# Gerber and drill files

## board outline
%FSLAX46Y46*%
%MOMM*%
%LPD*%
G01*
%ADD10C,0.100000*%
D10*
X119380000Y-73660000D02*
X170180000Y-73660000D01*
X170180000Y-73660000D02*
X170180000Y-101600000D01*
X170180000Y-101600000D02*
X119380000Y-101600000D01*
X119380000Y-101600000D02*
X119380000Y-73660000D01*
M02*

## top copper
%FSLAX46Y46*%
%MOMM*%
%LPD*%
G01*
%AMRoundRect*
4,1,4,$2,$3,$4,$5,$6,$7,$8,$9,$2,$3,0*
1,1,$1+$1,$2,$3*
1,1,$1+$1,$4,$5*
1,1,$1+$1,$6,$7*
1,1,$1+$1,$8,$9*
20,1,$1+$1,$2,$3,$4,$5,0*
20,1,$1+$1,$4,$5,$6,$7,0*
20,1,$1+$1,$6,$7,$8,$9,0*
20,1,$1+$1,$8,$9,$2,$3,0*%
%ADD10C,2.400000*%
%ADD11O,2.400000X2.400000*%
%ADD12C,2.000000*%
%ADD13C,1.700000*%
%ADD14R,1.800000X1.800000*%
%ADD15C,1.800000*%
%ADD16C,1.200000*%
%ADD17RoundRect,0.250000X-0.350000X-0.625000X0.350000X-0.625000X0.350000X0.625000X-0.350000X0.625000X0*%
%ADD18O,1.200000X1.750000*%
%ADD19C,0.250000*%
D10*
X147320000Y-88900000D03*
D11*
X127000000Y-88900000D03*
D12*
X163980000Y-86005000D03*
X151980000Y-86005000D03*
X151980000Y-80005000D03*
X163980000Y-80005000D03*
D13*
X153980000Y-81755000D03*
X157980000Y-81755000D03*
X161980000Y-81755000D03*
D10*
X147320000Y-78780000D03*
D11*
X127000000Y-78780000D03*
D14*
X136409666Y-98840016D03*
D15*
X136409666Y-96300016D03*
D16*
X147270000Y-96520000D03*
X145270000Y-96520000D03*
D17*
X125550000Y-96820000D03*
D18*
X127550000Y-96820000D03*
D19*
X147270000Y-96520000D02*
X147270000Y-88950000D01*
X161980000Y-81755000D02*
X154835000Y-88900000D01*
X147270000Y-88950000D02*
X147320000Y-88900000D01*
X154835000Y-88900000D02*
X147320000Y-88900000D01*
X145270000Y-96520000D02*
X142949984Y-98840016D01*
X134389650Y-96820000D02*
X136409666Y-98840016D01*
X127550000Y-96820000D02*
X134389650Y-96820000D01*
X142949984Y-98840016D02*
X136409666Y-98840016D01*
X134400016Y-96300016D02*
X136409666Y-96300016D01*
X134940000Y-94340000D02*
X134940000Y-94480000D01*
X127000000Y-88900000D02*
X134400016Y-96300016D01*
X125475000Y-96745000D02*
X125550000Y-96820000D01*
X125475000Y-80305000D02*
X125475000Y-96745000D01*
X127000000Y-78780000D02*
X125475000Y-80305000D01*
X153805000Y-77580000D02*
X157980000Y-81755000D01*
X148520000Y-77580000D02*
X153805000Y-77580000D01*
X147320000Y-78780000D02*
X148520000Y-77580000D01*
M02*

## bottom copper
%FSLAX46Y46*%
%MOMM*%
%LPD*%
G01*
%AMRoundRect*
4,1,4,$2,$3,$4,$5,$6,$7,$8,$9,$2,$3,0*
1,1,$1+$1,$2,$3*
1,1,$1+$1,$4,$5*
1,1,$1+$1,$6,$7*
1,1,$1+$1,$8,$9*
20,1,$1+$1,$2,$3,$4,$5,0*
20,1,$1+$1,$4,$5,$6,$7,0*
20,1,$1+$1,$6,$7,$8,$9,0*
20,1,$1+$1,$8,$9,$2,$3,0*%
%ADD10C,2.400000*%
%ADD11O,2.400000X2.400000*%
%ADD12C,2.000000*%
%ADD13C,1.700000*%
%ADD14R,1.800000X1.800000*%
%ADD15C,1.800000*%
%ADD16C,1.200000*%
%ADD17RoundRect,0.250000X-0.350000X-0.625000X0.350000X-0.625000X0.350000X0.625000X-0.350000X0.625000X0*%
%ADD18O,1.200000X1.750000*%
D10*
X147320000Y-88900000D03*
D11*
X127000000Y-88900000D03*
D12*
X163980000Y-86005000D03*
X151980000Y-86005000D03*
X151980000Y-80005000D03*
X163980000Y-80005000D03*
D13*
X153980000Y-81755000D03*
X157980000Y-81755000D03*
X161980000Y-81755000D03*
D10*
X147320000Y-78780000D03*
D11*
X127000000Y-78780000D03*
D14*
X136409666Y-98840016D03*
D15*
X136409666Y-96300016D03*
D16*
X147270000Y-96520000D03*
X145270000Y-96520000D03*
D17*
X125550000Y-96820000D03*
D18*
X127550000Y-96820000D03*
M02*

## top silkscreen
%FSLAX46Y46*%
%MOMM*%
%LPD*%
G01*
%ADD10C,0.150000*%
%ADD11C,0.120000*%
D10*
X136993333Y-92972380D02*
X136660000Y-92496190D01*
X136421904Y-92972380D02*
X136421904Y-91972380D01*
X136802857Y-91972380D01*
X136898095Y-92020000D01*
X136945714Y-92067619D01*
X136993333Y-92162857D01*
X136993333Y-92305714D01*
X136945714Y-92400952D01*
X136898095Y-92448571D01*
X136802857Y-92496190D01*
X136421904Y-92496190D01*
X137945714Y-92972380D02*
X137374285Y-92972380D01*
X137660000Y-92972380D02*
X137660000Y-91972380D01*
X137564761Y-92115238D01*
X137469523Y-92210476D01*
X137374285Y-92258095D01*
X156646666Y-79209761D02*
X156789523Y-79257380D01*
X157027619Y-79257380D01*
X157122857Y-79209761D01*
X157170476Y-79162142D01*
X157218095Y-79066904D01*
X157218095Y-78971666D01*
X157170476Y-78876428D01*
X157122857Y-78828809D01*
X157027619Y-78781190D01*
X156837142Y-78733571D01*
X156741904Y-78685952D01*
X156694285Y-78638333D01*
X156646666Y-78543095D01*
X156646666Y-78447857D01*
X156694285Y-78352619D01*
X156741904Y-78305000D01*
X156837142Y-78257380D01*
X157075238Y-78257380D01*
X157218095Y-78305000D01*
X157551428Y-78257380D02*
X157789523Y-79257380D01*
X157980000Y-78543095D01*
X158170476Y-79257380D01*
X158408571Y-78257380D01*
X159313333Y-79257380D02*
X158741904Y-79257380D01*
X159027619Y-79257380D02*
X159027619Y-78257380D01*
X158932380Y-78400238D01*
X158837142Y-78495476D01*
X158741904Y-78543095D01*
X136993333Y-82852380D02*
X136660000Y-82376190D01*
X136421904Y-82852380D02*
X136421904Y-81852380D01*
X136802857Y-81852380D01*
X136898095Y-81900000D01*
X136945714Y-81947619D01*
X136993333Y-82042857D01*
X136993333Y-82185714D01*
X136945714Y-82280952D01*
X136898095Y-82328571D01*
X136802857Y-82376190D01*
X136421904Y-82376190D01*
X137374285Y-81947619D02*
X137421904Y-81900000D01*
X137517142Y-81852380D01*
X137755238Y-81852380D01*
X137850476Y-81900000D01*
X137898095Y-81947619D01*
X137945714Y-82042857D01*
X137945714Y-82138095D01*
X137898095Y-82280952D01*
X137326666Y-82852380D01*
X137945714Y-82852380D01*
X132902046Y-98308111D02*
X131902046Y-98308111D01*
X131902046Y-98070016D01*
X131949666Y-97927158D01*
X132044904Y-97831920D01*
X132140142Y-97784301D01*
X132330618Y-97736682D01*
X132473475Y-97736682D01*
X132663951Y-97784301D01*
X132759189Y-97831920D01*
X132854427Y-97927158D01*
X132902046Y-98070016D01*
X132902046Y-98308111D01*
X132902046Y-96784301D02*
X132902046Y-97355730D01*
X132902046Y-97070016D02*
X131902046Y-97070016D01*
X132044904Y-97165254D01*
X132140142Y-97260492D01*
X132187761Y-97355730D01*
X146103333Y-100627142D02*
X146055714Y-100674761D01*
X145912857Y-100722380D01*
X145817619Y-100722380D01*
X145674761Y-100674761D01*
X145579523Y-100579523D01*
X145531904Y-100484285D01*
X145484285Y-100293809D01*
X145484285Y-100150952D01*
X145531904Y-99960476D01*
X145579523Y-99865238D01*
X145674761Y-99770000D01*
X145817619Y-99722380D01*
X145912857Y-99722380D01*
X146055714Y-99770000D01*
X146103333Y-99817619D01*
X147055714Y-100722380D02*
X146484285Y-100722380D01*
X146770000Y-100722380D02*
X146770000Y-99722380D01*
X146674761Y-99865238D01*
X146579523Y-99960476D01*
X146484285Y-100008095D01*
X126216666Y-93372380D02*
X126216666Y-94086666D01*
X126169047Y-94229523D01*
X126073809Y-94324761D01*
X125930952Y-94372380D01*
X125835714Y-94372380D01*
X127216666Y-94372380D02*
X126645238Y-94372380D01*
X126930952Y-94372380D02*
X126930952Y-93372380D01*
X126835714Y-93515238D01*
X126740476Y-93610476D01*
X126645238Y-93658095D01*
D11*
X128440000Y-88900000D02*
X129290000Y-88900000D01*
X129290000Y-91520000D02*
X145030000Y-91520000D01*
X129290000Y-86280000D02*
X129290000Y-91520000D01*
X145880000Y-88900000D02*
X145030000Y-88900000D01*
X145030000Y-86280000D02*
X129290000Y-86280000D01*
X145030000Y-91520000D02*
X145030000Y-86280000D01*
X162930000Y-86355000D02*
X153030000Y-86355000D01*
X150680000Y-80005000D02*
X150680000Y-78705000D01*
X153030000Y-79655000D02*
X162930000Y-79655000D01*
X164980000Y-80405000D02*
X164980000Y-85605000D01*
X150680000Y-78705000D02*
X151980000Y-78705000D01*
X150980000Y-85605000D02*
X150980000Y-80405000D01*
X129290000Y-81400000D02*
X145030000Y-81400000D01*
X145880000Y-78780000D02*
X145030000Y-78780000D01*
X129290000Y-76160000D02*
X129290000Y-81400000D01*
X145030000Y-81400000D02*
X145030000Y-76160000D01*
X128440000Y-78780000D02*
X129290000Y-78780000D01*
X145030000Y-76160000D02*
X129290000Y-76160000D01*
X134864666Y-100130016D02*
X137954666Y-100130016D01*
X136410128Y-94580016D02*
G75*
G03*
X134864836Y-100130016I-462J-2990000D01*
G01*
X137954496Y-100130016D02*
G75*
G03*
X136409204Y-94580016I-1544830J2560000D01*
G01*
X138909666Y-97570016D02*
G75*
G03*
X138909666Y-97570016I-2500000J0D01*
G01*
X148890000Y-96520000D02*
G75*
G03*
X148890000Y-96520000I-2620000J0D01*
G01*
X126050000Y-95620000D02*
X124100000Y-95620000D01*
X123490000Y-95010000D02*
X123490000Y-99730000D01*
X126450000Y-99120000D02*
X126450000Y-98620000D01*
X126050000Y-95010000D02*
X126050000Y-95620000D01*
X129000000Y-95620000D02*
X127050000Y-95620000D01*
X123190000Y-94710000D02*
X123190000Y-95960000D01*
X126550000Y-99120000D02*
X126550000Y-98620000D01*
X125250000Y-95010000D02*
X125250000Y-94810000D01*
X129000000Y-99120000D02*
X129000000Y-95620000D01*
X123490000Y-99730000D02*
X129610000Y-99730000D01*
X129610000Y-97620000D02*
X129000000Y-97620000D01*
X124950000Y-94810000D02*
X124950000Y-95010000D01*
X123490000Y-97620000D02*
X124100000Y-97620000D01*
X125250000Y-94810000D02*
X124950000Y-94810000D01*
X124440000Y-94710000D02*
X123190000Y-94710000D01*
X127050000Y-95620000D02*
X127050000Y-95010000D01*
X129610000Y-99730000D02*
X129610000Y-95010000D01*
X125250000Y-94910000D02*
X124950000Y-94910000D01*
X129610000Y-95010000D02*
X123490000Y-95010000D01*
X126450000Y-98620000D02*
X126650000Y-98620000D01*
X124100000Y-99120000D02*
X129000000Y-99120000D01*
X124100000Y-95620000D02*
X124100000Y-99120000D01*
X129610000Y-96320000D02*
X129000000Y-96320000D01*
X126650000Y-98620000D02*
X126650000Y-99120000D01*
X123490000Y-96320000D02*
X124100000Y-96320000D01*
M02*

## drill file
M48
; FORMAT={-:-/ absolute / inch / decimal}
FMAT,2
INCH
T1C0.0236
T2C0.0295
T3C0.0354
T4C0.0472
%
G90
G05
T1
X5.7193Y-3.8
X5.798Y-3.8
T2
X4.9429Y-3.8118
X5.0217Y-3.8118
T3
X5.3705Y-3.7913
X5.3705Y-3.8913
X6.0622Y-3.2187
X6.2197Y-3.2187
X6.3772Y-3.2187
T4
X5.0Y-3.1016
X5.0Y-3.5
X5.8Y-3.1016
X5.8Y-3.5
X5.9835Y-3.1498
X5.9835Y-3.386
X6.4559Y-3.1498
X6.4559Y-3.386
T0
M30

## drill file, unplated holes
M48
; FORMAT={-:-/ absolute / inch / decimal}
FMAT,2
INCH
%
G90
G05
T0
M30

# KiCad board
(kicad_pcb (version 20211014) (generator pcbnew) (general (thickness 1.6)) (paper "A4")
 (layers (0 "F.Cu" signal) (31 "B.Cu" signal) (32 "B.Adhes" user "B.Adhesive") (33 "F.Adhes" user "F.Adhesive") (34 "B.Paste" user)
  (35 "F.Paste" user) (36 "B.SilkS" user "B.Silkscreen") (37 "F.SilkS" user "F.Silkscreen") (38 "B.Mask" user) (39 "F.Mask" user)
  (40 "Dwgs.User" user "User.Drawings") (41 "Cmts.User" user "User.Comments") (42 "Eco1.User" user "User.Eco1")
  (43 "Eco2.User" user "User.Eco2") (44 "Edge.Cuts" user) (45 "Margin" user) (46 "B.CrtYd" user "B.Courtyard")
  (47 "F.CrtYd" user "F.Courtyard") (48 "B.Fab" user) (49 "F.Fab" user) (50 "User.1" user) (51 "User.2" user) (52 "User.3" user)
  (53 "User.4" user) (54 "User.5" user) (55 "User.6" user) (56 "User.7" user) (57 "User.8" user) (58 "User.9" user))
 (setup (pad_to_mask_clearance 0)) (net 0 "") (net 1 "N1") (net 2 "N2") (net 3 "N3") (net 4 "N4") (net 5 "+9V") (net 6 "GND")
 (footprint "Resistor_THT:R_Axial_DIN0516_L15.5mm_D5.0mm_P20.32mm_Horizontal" (layer "F.Cu") (at 147.32 88.9 180)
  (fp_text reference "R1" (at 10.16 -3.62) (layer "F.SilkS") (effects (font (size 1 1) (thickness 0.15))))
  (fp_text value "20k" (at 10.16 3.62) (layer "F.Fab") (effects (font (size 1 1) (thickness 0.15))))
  (fp_line (start 18.88 0) (end 18.03 0) (layer "F.SilkS") (width 0.12))
  (fp_line (start 18.03 -2.62) (end 2.29 -2.62) (layer "F.SilkS") (width 0.12))
  (fp_line (start 18.03 2.62) (end 18.03 -2.62) (layer "F.SilkS") (width 0.12))
  (fp_line (start 1.44 0) (end 2.29 0) (layer "F.SilkS") (width 0.12))
  (fp_line (start 2.29 2.62) (end 18.03 2.62) (layer "F.SilkS") (width 0.12))
  (fp_line (start 2.29 -2.62) (end 2.29 2.62) (layer "F.SilkS") (width 0.12))
  (pad "1" thru_hole circle (at 0 0 180) (size 2.4 2.4) (drill 1.2) (layers *.Cu *.Mask) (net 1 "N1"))
  (pad "2" thru_hole oval (at 20.32 0 180) (size 2.4 2.4) (drill 1.2) (layers *.Cu *.Mask) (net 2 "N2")))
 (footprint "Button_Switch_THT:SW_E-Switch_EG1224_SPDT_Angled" (layer "F.Cu") (at 153.98 81.755)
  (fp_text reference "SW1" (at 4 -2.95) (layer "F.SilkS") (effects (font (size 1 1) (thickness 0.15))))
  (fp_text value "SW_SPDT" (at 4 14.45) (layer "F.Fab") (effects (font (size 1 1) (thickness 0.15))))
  (fp_line (start 8.95 4.6) (end -0.95 4.6) (layer "F.SilkS") (width 0.12))
  (fp_line (start -3.3 -1.75) (end -3.3 -3.05) (layer "F.SilkS") (width 0.12))
  (fp_line (start -0.95 -2.1) (end 8.95 -2.1) (layer "F.SilkS") (width 0.12))
  (fp_line (start 11 -1.35) (end 11 3.85) (layer "F.SilkS") (width 0.12))
  (fp_line (start -3.3 -3.05) (end -2 -3.05) (layer "F.SilkS") (width 0.12))
  (fp_line (start -3 3.85) (end -3 -1.35) (layer "F.SilkS") (width 0.12))
  (pad "" thru_hole circle (at 10 4.25) (size 2 2) (drill 1.2) (layers *.Cu *.Mask))
  (pad "" thru_hole circle (at -2 4.25) (size 2 2) (drill 1.2) (layers *.Cu *.Mask))
  (pad "" thru_hole circle (at -2 -1.75) (size 2 2) (drill 1.2) (layers *.Cu *.Mask))
  (pad "" thru_hole circle (at 10 -1.75) (size 2 2) (drill 1.2) (layers *.Cu *.Mask))
  (pad "1" thru_hole circle (at 0 0) (size 1.7 1.7) (drill 0.9) (layers *.Cu *.Mask) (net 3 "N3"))
  (pad "2" thru_hole circle (at 4 0) (size 1.7 1.7) (drill 0.9) (layers *.Cu *.Mask) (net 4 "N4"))
  (pad "3" thru_hole circle (at 8 0) (size 1.7 1.7) (drill 0.9) (layers *.Cu *.Mask) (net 1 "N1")))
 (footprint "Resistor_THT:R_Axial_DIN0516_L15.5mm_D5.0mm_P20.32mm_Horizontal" (layer "F.Cu") (at 147.32 78.78 180)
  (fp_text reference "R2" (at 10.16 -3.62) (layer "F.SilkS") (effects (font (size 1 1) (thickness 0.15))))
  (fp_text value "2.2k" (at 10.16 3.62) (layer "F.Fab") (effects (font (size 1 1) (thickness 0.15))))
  (fp_line (start 18.03 -2.62) (end 2.29 -2.62) (layer "F.SilkS") (width 0.12))
  (fp_line (start 1.44 0) (end 2.29 0) (layer "F.SilkS") (width 0.12))
  (fp_line (start 18.03 2.62) (end 18.03 -2.62) (layer "F.SilkS") (width 0.12))
  (fp_line (start 2.29 -2.62) (end 2.29 2.62) (layer "F.SilkS") (width 0.12))
  (fp_line (start 18.88 0) (end 18.03 0) (layer "F.SilkS") (width 0.12))
  (fp_line (start 2.29 2.62) (end 18.03 2.62) (layer "F.SilkS") (width 0.12))
  (pad "1" thru_hole circle (at 0 0 180) (size 2.4 2.4) (drill 1.2) (layers *.Cu *.Mask) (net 4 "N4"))
  (pad "2" thru_hole oval (at 20.32 0 180) (size 2.4 2.4) (drill 1.2) (layers *.Cu *.Mask) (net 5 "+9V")))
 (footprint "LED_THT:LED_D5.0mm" (layer "F.Cu") (at 136.409666 98.840016 90)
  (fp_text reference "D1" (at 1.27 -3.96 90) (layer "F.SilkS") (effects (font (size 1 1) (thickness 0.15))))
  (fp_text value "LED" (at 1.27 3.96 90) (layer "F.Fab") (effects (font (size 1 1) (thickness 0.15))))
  (fp_line (start -1.29 -1.545) (end -1.29 1.545) (layer "F.SilkS") (width 0.12))
  (fp_arc (start -1.29 -1.54483) (mid 2.072002 -2.880433) (end 4.26 0.000462) (layer "F.SilkS") (width 0.12))
  (fp_arc (start 4.26 -0.000462) (mid 2.072002 2.880433) (end -1.29 1.54483) (layer "F.SilkS") (width 0.12))
  (fp_circle (center 1.27 0) (end 3.77 0) (layer "F.SilkS") (width 0.12) (fill none))
  (pad "1" thru_hole rect (at 0 0 90) (size 1.8 1.8) (drill 0.9) (layers *.Cu *.Mask) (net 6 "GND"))
  (pad "2" thru_hole circle (at 2.54 0 90) (size 1.8 1.8) (drill 0.9) (layers *.Cu *.Mask) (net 2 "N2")))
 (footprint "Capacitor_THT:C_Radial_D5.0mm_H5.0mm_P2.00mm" (layer "F.Cu") (at 147.27 96.52 180)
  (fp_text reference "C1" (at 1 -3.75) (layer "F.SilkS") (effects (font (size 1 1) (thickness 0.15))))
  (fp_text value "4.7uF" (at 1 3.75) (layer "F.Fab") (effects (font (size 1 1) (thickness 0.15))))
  (fp_circle (center 1 0) (end 3.62 0) (layer "F.SilkS") (width 0.12) (fill none))
  (pad "1" thru_hole circle (at 0 0 180) (size 1.2 1.2) (drill 0.6) (layers *.Cu *.Mask) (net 1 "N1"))
  (pad "2" thru_hole circle (at 2 0 180) (size 1.2 1.2) (drill 0.6) (layers *.Cu *.Mask) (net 6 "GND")))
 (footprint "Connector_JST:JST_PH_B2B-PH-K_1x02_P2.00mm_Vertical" (layer "F.Cu") (at 125.55 96.82)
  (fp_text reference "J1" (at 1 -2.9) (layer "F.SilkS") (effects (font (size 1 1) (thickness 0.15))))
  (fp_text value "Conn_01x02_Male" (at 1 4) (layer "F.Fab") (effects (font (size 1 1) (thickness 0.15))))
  (fp_line (start 0.5 -1.2) (end -1.45 -1.2) (layer "F.SilkS") (width 0.12))
  (fp_line (start -2.06 -1.81) (end -2.06 2.91) (layer "F.SilkS") (width 0.12))
  (fp_line (start 0.9 2.3) (end 0.9 1.8) (layer "F.SilkS") (width 0.12))
  (fp_line (start 0.5 -1.81) (end 0.5 -1.2) (layer "F.SilkS") (width 0.12))
  (fp_line (start 3.45 -1.2) (end 1.5 -1.2) (layer "F.SilkS") (width 0.12))
  (fp_line (start -2.36 -2.11) (end -2.36 -0.86) (layer "F.SilkS") (width 0.12))
  (fp_line (start 1 2.3) (end 1 1.8) (layer "F.SilkS") (width 0.12))
  (fp_line (start -0.3 -1.81) (end -0.3 -2.01) (layer "F.SilkS") (width 0.12))
  (fp_line (start 3.45 2.3) (end 3.45 -1.2) (layer "F.SilkS") (width 0.12))
  (fp_line (start -2.06 2.91) (end 4.06 2.91) (layer "F.SilkS") (width 0.12))
  (fp_line (start 4.06 0.8) (end 3.45 0.8) (layer "F.SilkS") (width 0.12))
  (fp_line (start -0.6 -2.01) (end -0.6 -1.81) (layer "F.SilkS") (width 0.12))
  (fp_line (start -2.06 0.8) (end -1.45 0.8) (layer "F.SilkS") (width 0.12))
  (fp_line (start -0.3 -2.01) (end -0.6 -2.01) (layer "F.SilkS") (width 0.12))
  (fp_line (start -1.11 -2.11) (end -2.36 -2.11) (layer "F.SilkS") (width 0.12))
  (fp_line (start 1.5 -1.2) (end 1.5 -1.81) (layer "F.SilkS") (width 0.12))
  (fp_line (start 4.06 2.91) (end 4.06 -1.81) (layer "F.SilkS") (width 0.12))
  (fp_line (start -0.3 -1.91) (end -0.6 -1.91) (layer "F.SilkS") (width 0.12))
  (fp_line (start 4.06 -1.81) (end -2.06 -1.81) (layer "F.SilkS") (width 0.12))
  (fp_line (start 0.9 1.8) (end 1.1 1.8) (layer "F.SilkS") (width 0.12))
  (fp_line (start -1.45 2.3) (end 3.45 2.3) (layer "F.SilkS") (width 0.12))
  (fp_line (start -1.45 -1.2) (end -1.45 2.3) (layer "F.SilkS") (width 0.12))
  (fp_line (start 4.06 -0.5) (end 3.45 -0.5) (layer "F.SilkS") (width 0.12))
  (fp_line (start 1.1 1.8) (end 1.1 2.3) (layer "F.SilkS") (width 0.12))
  (fp_line (start -2.06 -0.5) (end -1.45 -0.5) (layer "F.SilkS") (width 0.12))
  (pad "1" thru_hole roundrect (at 0 0) (size 1.2 1.75) (drill 0.75) (layers *.Cu *.Mask) (roundrect_rratio 0.2083333333) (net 5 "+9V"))
  (pad "2" thru_hole oval (at 2 0) (size 1.2 1.75) (drill 0.75) (layers *.Cu *.Mask) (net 6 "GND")))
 (gr_rect (start 119.38 73.66) (end 170.18 101.6) (layer "Edge.Cuts") (width 0.1) (fill none))
 (segment (start 147.27 96.52) (end 147.27 88.95) (width 0.25) (layer "F.Cu") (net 1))
 (segment (start 161.98 81.755) (end 154.835 88.9) (width 0.25) (layer "F.Cu") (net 1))
 (segment (start 147.27 88.95) (end 147.32 88.9) (width 0.25) (layer "F.Cu") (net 1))
 (segment (start 154.835 88.9) (end 147.32 88.9) (width 0.25) (layer "F.Cu") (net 1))
 (segment (start 145.27 96.52) (end 142.949984 98.840016) (width 0.25) (layer "F.Cu") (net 6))
 (segment (start 134.38965 96.82) (end 136.409666 98.840016) (width 0.25) (layer "F.Cu") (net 6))
 (segment (start 127.55 96.82) (end 134.38965 96.82) (width 0.25) (layer "F.Cu") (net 6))
 (segment (start 142.949984 98.840016) (end 136.409666 98.840016) (width 0.25) (layer "F.Cu") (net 6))
 (segment (start 134.400016 96.300016) (end 136.409666 96.300016) (width 0.25) (layer "F.Cu") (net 2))
 (segment (start 134.94 94.34) (end 134.94 94.48) (width 0.25) (layer "F.Cu") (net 2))
 (segment (start 127 88.9) (end 134.400016 96.300016) (width 0.25) (layer "F.Cu") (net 2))
 (segment (start 125.475 96.745) (end 125.55 96.82) (width 0.25) (layer "F.Cu") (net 5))
 (segment (start 125.475 80.305) (end 125.475 96.745) (width 0.25) (layer "F.Cu") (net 5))
 (segment (start 127 78.78) (end 125.475 80.305) (width 0.25) (layer "F.Cu") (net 5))
 (segment (start 153.805 77.58) (end 157.98 81.755) (width 0.25) (layer "F.Cu") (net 4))
 (segment (start 148.52 77.58) (end 153.805 77.58) (width 0.25) (layer "F.Cu") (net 4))
 (segment (start 147.32 78.78) (end 148.52 77.58) (width 0.25) (layer "F.Cu") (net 4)))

